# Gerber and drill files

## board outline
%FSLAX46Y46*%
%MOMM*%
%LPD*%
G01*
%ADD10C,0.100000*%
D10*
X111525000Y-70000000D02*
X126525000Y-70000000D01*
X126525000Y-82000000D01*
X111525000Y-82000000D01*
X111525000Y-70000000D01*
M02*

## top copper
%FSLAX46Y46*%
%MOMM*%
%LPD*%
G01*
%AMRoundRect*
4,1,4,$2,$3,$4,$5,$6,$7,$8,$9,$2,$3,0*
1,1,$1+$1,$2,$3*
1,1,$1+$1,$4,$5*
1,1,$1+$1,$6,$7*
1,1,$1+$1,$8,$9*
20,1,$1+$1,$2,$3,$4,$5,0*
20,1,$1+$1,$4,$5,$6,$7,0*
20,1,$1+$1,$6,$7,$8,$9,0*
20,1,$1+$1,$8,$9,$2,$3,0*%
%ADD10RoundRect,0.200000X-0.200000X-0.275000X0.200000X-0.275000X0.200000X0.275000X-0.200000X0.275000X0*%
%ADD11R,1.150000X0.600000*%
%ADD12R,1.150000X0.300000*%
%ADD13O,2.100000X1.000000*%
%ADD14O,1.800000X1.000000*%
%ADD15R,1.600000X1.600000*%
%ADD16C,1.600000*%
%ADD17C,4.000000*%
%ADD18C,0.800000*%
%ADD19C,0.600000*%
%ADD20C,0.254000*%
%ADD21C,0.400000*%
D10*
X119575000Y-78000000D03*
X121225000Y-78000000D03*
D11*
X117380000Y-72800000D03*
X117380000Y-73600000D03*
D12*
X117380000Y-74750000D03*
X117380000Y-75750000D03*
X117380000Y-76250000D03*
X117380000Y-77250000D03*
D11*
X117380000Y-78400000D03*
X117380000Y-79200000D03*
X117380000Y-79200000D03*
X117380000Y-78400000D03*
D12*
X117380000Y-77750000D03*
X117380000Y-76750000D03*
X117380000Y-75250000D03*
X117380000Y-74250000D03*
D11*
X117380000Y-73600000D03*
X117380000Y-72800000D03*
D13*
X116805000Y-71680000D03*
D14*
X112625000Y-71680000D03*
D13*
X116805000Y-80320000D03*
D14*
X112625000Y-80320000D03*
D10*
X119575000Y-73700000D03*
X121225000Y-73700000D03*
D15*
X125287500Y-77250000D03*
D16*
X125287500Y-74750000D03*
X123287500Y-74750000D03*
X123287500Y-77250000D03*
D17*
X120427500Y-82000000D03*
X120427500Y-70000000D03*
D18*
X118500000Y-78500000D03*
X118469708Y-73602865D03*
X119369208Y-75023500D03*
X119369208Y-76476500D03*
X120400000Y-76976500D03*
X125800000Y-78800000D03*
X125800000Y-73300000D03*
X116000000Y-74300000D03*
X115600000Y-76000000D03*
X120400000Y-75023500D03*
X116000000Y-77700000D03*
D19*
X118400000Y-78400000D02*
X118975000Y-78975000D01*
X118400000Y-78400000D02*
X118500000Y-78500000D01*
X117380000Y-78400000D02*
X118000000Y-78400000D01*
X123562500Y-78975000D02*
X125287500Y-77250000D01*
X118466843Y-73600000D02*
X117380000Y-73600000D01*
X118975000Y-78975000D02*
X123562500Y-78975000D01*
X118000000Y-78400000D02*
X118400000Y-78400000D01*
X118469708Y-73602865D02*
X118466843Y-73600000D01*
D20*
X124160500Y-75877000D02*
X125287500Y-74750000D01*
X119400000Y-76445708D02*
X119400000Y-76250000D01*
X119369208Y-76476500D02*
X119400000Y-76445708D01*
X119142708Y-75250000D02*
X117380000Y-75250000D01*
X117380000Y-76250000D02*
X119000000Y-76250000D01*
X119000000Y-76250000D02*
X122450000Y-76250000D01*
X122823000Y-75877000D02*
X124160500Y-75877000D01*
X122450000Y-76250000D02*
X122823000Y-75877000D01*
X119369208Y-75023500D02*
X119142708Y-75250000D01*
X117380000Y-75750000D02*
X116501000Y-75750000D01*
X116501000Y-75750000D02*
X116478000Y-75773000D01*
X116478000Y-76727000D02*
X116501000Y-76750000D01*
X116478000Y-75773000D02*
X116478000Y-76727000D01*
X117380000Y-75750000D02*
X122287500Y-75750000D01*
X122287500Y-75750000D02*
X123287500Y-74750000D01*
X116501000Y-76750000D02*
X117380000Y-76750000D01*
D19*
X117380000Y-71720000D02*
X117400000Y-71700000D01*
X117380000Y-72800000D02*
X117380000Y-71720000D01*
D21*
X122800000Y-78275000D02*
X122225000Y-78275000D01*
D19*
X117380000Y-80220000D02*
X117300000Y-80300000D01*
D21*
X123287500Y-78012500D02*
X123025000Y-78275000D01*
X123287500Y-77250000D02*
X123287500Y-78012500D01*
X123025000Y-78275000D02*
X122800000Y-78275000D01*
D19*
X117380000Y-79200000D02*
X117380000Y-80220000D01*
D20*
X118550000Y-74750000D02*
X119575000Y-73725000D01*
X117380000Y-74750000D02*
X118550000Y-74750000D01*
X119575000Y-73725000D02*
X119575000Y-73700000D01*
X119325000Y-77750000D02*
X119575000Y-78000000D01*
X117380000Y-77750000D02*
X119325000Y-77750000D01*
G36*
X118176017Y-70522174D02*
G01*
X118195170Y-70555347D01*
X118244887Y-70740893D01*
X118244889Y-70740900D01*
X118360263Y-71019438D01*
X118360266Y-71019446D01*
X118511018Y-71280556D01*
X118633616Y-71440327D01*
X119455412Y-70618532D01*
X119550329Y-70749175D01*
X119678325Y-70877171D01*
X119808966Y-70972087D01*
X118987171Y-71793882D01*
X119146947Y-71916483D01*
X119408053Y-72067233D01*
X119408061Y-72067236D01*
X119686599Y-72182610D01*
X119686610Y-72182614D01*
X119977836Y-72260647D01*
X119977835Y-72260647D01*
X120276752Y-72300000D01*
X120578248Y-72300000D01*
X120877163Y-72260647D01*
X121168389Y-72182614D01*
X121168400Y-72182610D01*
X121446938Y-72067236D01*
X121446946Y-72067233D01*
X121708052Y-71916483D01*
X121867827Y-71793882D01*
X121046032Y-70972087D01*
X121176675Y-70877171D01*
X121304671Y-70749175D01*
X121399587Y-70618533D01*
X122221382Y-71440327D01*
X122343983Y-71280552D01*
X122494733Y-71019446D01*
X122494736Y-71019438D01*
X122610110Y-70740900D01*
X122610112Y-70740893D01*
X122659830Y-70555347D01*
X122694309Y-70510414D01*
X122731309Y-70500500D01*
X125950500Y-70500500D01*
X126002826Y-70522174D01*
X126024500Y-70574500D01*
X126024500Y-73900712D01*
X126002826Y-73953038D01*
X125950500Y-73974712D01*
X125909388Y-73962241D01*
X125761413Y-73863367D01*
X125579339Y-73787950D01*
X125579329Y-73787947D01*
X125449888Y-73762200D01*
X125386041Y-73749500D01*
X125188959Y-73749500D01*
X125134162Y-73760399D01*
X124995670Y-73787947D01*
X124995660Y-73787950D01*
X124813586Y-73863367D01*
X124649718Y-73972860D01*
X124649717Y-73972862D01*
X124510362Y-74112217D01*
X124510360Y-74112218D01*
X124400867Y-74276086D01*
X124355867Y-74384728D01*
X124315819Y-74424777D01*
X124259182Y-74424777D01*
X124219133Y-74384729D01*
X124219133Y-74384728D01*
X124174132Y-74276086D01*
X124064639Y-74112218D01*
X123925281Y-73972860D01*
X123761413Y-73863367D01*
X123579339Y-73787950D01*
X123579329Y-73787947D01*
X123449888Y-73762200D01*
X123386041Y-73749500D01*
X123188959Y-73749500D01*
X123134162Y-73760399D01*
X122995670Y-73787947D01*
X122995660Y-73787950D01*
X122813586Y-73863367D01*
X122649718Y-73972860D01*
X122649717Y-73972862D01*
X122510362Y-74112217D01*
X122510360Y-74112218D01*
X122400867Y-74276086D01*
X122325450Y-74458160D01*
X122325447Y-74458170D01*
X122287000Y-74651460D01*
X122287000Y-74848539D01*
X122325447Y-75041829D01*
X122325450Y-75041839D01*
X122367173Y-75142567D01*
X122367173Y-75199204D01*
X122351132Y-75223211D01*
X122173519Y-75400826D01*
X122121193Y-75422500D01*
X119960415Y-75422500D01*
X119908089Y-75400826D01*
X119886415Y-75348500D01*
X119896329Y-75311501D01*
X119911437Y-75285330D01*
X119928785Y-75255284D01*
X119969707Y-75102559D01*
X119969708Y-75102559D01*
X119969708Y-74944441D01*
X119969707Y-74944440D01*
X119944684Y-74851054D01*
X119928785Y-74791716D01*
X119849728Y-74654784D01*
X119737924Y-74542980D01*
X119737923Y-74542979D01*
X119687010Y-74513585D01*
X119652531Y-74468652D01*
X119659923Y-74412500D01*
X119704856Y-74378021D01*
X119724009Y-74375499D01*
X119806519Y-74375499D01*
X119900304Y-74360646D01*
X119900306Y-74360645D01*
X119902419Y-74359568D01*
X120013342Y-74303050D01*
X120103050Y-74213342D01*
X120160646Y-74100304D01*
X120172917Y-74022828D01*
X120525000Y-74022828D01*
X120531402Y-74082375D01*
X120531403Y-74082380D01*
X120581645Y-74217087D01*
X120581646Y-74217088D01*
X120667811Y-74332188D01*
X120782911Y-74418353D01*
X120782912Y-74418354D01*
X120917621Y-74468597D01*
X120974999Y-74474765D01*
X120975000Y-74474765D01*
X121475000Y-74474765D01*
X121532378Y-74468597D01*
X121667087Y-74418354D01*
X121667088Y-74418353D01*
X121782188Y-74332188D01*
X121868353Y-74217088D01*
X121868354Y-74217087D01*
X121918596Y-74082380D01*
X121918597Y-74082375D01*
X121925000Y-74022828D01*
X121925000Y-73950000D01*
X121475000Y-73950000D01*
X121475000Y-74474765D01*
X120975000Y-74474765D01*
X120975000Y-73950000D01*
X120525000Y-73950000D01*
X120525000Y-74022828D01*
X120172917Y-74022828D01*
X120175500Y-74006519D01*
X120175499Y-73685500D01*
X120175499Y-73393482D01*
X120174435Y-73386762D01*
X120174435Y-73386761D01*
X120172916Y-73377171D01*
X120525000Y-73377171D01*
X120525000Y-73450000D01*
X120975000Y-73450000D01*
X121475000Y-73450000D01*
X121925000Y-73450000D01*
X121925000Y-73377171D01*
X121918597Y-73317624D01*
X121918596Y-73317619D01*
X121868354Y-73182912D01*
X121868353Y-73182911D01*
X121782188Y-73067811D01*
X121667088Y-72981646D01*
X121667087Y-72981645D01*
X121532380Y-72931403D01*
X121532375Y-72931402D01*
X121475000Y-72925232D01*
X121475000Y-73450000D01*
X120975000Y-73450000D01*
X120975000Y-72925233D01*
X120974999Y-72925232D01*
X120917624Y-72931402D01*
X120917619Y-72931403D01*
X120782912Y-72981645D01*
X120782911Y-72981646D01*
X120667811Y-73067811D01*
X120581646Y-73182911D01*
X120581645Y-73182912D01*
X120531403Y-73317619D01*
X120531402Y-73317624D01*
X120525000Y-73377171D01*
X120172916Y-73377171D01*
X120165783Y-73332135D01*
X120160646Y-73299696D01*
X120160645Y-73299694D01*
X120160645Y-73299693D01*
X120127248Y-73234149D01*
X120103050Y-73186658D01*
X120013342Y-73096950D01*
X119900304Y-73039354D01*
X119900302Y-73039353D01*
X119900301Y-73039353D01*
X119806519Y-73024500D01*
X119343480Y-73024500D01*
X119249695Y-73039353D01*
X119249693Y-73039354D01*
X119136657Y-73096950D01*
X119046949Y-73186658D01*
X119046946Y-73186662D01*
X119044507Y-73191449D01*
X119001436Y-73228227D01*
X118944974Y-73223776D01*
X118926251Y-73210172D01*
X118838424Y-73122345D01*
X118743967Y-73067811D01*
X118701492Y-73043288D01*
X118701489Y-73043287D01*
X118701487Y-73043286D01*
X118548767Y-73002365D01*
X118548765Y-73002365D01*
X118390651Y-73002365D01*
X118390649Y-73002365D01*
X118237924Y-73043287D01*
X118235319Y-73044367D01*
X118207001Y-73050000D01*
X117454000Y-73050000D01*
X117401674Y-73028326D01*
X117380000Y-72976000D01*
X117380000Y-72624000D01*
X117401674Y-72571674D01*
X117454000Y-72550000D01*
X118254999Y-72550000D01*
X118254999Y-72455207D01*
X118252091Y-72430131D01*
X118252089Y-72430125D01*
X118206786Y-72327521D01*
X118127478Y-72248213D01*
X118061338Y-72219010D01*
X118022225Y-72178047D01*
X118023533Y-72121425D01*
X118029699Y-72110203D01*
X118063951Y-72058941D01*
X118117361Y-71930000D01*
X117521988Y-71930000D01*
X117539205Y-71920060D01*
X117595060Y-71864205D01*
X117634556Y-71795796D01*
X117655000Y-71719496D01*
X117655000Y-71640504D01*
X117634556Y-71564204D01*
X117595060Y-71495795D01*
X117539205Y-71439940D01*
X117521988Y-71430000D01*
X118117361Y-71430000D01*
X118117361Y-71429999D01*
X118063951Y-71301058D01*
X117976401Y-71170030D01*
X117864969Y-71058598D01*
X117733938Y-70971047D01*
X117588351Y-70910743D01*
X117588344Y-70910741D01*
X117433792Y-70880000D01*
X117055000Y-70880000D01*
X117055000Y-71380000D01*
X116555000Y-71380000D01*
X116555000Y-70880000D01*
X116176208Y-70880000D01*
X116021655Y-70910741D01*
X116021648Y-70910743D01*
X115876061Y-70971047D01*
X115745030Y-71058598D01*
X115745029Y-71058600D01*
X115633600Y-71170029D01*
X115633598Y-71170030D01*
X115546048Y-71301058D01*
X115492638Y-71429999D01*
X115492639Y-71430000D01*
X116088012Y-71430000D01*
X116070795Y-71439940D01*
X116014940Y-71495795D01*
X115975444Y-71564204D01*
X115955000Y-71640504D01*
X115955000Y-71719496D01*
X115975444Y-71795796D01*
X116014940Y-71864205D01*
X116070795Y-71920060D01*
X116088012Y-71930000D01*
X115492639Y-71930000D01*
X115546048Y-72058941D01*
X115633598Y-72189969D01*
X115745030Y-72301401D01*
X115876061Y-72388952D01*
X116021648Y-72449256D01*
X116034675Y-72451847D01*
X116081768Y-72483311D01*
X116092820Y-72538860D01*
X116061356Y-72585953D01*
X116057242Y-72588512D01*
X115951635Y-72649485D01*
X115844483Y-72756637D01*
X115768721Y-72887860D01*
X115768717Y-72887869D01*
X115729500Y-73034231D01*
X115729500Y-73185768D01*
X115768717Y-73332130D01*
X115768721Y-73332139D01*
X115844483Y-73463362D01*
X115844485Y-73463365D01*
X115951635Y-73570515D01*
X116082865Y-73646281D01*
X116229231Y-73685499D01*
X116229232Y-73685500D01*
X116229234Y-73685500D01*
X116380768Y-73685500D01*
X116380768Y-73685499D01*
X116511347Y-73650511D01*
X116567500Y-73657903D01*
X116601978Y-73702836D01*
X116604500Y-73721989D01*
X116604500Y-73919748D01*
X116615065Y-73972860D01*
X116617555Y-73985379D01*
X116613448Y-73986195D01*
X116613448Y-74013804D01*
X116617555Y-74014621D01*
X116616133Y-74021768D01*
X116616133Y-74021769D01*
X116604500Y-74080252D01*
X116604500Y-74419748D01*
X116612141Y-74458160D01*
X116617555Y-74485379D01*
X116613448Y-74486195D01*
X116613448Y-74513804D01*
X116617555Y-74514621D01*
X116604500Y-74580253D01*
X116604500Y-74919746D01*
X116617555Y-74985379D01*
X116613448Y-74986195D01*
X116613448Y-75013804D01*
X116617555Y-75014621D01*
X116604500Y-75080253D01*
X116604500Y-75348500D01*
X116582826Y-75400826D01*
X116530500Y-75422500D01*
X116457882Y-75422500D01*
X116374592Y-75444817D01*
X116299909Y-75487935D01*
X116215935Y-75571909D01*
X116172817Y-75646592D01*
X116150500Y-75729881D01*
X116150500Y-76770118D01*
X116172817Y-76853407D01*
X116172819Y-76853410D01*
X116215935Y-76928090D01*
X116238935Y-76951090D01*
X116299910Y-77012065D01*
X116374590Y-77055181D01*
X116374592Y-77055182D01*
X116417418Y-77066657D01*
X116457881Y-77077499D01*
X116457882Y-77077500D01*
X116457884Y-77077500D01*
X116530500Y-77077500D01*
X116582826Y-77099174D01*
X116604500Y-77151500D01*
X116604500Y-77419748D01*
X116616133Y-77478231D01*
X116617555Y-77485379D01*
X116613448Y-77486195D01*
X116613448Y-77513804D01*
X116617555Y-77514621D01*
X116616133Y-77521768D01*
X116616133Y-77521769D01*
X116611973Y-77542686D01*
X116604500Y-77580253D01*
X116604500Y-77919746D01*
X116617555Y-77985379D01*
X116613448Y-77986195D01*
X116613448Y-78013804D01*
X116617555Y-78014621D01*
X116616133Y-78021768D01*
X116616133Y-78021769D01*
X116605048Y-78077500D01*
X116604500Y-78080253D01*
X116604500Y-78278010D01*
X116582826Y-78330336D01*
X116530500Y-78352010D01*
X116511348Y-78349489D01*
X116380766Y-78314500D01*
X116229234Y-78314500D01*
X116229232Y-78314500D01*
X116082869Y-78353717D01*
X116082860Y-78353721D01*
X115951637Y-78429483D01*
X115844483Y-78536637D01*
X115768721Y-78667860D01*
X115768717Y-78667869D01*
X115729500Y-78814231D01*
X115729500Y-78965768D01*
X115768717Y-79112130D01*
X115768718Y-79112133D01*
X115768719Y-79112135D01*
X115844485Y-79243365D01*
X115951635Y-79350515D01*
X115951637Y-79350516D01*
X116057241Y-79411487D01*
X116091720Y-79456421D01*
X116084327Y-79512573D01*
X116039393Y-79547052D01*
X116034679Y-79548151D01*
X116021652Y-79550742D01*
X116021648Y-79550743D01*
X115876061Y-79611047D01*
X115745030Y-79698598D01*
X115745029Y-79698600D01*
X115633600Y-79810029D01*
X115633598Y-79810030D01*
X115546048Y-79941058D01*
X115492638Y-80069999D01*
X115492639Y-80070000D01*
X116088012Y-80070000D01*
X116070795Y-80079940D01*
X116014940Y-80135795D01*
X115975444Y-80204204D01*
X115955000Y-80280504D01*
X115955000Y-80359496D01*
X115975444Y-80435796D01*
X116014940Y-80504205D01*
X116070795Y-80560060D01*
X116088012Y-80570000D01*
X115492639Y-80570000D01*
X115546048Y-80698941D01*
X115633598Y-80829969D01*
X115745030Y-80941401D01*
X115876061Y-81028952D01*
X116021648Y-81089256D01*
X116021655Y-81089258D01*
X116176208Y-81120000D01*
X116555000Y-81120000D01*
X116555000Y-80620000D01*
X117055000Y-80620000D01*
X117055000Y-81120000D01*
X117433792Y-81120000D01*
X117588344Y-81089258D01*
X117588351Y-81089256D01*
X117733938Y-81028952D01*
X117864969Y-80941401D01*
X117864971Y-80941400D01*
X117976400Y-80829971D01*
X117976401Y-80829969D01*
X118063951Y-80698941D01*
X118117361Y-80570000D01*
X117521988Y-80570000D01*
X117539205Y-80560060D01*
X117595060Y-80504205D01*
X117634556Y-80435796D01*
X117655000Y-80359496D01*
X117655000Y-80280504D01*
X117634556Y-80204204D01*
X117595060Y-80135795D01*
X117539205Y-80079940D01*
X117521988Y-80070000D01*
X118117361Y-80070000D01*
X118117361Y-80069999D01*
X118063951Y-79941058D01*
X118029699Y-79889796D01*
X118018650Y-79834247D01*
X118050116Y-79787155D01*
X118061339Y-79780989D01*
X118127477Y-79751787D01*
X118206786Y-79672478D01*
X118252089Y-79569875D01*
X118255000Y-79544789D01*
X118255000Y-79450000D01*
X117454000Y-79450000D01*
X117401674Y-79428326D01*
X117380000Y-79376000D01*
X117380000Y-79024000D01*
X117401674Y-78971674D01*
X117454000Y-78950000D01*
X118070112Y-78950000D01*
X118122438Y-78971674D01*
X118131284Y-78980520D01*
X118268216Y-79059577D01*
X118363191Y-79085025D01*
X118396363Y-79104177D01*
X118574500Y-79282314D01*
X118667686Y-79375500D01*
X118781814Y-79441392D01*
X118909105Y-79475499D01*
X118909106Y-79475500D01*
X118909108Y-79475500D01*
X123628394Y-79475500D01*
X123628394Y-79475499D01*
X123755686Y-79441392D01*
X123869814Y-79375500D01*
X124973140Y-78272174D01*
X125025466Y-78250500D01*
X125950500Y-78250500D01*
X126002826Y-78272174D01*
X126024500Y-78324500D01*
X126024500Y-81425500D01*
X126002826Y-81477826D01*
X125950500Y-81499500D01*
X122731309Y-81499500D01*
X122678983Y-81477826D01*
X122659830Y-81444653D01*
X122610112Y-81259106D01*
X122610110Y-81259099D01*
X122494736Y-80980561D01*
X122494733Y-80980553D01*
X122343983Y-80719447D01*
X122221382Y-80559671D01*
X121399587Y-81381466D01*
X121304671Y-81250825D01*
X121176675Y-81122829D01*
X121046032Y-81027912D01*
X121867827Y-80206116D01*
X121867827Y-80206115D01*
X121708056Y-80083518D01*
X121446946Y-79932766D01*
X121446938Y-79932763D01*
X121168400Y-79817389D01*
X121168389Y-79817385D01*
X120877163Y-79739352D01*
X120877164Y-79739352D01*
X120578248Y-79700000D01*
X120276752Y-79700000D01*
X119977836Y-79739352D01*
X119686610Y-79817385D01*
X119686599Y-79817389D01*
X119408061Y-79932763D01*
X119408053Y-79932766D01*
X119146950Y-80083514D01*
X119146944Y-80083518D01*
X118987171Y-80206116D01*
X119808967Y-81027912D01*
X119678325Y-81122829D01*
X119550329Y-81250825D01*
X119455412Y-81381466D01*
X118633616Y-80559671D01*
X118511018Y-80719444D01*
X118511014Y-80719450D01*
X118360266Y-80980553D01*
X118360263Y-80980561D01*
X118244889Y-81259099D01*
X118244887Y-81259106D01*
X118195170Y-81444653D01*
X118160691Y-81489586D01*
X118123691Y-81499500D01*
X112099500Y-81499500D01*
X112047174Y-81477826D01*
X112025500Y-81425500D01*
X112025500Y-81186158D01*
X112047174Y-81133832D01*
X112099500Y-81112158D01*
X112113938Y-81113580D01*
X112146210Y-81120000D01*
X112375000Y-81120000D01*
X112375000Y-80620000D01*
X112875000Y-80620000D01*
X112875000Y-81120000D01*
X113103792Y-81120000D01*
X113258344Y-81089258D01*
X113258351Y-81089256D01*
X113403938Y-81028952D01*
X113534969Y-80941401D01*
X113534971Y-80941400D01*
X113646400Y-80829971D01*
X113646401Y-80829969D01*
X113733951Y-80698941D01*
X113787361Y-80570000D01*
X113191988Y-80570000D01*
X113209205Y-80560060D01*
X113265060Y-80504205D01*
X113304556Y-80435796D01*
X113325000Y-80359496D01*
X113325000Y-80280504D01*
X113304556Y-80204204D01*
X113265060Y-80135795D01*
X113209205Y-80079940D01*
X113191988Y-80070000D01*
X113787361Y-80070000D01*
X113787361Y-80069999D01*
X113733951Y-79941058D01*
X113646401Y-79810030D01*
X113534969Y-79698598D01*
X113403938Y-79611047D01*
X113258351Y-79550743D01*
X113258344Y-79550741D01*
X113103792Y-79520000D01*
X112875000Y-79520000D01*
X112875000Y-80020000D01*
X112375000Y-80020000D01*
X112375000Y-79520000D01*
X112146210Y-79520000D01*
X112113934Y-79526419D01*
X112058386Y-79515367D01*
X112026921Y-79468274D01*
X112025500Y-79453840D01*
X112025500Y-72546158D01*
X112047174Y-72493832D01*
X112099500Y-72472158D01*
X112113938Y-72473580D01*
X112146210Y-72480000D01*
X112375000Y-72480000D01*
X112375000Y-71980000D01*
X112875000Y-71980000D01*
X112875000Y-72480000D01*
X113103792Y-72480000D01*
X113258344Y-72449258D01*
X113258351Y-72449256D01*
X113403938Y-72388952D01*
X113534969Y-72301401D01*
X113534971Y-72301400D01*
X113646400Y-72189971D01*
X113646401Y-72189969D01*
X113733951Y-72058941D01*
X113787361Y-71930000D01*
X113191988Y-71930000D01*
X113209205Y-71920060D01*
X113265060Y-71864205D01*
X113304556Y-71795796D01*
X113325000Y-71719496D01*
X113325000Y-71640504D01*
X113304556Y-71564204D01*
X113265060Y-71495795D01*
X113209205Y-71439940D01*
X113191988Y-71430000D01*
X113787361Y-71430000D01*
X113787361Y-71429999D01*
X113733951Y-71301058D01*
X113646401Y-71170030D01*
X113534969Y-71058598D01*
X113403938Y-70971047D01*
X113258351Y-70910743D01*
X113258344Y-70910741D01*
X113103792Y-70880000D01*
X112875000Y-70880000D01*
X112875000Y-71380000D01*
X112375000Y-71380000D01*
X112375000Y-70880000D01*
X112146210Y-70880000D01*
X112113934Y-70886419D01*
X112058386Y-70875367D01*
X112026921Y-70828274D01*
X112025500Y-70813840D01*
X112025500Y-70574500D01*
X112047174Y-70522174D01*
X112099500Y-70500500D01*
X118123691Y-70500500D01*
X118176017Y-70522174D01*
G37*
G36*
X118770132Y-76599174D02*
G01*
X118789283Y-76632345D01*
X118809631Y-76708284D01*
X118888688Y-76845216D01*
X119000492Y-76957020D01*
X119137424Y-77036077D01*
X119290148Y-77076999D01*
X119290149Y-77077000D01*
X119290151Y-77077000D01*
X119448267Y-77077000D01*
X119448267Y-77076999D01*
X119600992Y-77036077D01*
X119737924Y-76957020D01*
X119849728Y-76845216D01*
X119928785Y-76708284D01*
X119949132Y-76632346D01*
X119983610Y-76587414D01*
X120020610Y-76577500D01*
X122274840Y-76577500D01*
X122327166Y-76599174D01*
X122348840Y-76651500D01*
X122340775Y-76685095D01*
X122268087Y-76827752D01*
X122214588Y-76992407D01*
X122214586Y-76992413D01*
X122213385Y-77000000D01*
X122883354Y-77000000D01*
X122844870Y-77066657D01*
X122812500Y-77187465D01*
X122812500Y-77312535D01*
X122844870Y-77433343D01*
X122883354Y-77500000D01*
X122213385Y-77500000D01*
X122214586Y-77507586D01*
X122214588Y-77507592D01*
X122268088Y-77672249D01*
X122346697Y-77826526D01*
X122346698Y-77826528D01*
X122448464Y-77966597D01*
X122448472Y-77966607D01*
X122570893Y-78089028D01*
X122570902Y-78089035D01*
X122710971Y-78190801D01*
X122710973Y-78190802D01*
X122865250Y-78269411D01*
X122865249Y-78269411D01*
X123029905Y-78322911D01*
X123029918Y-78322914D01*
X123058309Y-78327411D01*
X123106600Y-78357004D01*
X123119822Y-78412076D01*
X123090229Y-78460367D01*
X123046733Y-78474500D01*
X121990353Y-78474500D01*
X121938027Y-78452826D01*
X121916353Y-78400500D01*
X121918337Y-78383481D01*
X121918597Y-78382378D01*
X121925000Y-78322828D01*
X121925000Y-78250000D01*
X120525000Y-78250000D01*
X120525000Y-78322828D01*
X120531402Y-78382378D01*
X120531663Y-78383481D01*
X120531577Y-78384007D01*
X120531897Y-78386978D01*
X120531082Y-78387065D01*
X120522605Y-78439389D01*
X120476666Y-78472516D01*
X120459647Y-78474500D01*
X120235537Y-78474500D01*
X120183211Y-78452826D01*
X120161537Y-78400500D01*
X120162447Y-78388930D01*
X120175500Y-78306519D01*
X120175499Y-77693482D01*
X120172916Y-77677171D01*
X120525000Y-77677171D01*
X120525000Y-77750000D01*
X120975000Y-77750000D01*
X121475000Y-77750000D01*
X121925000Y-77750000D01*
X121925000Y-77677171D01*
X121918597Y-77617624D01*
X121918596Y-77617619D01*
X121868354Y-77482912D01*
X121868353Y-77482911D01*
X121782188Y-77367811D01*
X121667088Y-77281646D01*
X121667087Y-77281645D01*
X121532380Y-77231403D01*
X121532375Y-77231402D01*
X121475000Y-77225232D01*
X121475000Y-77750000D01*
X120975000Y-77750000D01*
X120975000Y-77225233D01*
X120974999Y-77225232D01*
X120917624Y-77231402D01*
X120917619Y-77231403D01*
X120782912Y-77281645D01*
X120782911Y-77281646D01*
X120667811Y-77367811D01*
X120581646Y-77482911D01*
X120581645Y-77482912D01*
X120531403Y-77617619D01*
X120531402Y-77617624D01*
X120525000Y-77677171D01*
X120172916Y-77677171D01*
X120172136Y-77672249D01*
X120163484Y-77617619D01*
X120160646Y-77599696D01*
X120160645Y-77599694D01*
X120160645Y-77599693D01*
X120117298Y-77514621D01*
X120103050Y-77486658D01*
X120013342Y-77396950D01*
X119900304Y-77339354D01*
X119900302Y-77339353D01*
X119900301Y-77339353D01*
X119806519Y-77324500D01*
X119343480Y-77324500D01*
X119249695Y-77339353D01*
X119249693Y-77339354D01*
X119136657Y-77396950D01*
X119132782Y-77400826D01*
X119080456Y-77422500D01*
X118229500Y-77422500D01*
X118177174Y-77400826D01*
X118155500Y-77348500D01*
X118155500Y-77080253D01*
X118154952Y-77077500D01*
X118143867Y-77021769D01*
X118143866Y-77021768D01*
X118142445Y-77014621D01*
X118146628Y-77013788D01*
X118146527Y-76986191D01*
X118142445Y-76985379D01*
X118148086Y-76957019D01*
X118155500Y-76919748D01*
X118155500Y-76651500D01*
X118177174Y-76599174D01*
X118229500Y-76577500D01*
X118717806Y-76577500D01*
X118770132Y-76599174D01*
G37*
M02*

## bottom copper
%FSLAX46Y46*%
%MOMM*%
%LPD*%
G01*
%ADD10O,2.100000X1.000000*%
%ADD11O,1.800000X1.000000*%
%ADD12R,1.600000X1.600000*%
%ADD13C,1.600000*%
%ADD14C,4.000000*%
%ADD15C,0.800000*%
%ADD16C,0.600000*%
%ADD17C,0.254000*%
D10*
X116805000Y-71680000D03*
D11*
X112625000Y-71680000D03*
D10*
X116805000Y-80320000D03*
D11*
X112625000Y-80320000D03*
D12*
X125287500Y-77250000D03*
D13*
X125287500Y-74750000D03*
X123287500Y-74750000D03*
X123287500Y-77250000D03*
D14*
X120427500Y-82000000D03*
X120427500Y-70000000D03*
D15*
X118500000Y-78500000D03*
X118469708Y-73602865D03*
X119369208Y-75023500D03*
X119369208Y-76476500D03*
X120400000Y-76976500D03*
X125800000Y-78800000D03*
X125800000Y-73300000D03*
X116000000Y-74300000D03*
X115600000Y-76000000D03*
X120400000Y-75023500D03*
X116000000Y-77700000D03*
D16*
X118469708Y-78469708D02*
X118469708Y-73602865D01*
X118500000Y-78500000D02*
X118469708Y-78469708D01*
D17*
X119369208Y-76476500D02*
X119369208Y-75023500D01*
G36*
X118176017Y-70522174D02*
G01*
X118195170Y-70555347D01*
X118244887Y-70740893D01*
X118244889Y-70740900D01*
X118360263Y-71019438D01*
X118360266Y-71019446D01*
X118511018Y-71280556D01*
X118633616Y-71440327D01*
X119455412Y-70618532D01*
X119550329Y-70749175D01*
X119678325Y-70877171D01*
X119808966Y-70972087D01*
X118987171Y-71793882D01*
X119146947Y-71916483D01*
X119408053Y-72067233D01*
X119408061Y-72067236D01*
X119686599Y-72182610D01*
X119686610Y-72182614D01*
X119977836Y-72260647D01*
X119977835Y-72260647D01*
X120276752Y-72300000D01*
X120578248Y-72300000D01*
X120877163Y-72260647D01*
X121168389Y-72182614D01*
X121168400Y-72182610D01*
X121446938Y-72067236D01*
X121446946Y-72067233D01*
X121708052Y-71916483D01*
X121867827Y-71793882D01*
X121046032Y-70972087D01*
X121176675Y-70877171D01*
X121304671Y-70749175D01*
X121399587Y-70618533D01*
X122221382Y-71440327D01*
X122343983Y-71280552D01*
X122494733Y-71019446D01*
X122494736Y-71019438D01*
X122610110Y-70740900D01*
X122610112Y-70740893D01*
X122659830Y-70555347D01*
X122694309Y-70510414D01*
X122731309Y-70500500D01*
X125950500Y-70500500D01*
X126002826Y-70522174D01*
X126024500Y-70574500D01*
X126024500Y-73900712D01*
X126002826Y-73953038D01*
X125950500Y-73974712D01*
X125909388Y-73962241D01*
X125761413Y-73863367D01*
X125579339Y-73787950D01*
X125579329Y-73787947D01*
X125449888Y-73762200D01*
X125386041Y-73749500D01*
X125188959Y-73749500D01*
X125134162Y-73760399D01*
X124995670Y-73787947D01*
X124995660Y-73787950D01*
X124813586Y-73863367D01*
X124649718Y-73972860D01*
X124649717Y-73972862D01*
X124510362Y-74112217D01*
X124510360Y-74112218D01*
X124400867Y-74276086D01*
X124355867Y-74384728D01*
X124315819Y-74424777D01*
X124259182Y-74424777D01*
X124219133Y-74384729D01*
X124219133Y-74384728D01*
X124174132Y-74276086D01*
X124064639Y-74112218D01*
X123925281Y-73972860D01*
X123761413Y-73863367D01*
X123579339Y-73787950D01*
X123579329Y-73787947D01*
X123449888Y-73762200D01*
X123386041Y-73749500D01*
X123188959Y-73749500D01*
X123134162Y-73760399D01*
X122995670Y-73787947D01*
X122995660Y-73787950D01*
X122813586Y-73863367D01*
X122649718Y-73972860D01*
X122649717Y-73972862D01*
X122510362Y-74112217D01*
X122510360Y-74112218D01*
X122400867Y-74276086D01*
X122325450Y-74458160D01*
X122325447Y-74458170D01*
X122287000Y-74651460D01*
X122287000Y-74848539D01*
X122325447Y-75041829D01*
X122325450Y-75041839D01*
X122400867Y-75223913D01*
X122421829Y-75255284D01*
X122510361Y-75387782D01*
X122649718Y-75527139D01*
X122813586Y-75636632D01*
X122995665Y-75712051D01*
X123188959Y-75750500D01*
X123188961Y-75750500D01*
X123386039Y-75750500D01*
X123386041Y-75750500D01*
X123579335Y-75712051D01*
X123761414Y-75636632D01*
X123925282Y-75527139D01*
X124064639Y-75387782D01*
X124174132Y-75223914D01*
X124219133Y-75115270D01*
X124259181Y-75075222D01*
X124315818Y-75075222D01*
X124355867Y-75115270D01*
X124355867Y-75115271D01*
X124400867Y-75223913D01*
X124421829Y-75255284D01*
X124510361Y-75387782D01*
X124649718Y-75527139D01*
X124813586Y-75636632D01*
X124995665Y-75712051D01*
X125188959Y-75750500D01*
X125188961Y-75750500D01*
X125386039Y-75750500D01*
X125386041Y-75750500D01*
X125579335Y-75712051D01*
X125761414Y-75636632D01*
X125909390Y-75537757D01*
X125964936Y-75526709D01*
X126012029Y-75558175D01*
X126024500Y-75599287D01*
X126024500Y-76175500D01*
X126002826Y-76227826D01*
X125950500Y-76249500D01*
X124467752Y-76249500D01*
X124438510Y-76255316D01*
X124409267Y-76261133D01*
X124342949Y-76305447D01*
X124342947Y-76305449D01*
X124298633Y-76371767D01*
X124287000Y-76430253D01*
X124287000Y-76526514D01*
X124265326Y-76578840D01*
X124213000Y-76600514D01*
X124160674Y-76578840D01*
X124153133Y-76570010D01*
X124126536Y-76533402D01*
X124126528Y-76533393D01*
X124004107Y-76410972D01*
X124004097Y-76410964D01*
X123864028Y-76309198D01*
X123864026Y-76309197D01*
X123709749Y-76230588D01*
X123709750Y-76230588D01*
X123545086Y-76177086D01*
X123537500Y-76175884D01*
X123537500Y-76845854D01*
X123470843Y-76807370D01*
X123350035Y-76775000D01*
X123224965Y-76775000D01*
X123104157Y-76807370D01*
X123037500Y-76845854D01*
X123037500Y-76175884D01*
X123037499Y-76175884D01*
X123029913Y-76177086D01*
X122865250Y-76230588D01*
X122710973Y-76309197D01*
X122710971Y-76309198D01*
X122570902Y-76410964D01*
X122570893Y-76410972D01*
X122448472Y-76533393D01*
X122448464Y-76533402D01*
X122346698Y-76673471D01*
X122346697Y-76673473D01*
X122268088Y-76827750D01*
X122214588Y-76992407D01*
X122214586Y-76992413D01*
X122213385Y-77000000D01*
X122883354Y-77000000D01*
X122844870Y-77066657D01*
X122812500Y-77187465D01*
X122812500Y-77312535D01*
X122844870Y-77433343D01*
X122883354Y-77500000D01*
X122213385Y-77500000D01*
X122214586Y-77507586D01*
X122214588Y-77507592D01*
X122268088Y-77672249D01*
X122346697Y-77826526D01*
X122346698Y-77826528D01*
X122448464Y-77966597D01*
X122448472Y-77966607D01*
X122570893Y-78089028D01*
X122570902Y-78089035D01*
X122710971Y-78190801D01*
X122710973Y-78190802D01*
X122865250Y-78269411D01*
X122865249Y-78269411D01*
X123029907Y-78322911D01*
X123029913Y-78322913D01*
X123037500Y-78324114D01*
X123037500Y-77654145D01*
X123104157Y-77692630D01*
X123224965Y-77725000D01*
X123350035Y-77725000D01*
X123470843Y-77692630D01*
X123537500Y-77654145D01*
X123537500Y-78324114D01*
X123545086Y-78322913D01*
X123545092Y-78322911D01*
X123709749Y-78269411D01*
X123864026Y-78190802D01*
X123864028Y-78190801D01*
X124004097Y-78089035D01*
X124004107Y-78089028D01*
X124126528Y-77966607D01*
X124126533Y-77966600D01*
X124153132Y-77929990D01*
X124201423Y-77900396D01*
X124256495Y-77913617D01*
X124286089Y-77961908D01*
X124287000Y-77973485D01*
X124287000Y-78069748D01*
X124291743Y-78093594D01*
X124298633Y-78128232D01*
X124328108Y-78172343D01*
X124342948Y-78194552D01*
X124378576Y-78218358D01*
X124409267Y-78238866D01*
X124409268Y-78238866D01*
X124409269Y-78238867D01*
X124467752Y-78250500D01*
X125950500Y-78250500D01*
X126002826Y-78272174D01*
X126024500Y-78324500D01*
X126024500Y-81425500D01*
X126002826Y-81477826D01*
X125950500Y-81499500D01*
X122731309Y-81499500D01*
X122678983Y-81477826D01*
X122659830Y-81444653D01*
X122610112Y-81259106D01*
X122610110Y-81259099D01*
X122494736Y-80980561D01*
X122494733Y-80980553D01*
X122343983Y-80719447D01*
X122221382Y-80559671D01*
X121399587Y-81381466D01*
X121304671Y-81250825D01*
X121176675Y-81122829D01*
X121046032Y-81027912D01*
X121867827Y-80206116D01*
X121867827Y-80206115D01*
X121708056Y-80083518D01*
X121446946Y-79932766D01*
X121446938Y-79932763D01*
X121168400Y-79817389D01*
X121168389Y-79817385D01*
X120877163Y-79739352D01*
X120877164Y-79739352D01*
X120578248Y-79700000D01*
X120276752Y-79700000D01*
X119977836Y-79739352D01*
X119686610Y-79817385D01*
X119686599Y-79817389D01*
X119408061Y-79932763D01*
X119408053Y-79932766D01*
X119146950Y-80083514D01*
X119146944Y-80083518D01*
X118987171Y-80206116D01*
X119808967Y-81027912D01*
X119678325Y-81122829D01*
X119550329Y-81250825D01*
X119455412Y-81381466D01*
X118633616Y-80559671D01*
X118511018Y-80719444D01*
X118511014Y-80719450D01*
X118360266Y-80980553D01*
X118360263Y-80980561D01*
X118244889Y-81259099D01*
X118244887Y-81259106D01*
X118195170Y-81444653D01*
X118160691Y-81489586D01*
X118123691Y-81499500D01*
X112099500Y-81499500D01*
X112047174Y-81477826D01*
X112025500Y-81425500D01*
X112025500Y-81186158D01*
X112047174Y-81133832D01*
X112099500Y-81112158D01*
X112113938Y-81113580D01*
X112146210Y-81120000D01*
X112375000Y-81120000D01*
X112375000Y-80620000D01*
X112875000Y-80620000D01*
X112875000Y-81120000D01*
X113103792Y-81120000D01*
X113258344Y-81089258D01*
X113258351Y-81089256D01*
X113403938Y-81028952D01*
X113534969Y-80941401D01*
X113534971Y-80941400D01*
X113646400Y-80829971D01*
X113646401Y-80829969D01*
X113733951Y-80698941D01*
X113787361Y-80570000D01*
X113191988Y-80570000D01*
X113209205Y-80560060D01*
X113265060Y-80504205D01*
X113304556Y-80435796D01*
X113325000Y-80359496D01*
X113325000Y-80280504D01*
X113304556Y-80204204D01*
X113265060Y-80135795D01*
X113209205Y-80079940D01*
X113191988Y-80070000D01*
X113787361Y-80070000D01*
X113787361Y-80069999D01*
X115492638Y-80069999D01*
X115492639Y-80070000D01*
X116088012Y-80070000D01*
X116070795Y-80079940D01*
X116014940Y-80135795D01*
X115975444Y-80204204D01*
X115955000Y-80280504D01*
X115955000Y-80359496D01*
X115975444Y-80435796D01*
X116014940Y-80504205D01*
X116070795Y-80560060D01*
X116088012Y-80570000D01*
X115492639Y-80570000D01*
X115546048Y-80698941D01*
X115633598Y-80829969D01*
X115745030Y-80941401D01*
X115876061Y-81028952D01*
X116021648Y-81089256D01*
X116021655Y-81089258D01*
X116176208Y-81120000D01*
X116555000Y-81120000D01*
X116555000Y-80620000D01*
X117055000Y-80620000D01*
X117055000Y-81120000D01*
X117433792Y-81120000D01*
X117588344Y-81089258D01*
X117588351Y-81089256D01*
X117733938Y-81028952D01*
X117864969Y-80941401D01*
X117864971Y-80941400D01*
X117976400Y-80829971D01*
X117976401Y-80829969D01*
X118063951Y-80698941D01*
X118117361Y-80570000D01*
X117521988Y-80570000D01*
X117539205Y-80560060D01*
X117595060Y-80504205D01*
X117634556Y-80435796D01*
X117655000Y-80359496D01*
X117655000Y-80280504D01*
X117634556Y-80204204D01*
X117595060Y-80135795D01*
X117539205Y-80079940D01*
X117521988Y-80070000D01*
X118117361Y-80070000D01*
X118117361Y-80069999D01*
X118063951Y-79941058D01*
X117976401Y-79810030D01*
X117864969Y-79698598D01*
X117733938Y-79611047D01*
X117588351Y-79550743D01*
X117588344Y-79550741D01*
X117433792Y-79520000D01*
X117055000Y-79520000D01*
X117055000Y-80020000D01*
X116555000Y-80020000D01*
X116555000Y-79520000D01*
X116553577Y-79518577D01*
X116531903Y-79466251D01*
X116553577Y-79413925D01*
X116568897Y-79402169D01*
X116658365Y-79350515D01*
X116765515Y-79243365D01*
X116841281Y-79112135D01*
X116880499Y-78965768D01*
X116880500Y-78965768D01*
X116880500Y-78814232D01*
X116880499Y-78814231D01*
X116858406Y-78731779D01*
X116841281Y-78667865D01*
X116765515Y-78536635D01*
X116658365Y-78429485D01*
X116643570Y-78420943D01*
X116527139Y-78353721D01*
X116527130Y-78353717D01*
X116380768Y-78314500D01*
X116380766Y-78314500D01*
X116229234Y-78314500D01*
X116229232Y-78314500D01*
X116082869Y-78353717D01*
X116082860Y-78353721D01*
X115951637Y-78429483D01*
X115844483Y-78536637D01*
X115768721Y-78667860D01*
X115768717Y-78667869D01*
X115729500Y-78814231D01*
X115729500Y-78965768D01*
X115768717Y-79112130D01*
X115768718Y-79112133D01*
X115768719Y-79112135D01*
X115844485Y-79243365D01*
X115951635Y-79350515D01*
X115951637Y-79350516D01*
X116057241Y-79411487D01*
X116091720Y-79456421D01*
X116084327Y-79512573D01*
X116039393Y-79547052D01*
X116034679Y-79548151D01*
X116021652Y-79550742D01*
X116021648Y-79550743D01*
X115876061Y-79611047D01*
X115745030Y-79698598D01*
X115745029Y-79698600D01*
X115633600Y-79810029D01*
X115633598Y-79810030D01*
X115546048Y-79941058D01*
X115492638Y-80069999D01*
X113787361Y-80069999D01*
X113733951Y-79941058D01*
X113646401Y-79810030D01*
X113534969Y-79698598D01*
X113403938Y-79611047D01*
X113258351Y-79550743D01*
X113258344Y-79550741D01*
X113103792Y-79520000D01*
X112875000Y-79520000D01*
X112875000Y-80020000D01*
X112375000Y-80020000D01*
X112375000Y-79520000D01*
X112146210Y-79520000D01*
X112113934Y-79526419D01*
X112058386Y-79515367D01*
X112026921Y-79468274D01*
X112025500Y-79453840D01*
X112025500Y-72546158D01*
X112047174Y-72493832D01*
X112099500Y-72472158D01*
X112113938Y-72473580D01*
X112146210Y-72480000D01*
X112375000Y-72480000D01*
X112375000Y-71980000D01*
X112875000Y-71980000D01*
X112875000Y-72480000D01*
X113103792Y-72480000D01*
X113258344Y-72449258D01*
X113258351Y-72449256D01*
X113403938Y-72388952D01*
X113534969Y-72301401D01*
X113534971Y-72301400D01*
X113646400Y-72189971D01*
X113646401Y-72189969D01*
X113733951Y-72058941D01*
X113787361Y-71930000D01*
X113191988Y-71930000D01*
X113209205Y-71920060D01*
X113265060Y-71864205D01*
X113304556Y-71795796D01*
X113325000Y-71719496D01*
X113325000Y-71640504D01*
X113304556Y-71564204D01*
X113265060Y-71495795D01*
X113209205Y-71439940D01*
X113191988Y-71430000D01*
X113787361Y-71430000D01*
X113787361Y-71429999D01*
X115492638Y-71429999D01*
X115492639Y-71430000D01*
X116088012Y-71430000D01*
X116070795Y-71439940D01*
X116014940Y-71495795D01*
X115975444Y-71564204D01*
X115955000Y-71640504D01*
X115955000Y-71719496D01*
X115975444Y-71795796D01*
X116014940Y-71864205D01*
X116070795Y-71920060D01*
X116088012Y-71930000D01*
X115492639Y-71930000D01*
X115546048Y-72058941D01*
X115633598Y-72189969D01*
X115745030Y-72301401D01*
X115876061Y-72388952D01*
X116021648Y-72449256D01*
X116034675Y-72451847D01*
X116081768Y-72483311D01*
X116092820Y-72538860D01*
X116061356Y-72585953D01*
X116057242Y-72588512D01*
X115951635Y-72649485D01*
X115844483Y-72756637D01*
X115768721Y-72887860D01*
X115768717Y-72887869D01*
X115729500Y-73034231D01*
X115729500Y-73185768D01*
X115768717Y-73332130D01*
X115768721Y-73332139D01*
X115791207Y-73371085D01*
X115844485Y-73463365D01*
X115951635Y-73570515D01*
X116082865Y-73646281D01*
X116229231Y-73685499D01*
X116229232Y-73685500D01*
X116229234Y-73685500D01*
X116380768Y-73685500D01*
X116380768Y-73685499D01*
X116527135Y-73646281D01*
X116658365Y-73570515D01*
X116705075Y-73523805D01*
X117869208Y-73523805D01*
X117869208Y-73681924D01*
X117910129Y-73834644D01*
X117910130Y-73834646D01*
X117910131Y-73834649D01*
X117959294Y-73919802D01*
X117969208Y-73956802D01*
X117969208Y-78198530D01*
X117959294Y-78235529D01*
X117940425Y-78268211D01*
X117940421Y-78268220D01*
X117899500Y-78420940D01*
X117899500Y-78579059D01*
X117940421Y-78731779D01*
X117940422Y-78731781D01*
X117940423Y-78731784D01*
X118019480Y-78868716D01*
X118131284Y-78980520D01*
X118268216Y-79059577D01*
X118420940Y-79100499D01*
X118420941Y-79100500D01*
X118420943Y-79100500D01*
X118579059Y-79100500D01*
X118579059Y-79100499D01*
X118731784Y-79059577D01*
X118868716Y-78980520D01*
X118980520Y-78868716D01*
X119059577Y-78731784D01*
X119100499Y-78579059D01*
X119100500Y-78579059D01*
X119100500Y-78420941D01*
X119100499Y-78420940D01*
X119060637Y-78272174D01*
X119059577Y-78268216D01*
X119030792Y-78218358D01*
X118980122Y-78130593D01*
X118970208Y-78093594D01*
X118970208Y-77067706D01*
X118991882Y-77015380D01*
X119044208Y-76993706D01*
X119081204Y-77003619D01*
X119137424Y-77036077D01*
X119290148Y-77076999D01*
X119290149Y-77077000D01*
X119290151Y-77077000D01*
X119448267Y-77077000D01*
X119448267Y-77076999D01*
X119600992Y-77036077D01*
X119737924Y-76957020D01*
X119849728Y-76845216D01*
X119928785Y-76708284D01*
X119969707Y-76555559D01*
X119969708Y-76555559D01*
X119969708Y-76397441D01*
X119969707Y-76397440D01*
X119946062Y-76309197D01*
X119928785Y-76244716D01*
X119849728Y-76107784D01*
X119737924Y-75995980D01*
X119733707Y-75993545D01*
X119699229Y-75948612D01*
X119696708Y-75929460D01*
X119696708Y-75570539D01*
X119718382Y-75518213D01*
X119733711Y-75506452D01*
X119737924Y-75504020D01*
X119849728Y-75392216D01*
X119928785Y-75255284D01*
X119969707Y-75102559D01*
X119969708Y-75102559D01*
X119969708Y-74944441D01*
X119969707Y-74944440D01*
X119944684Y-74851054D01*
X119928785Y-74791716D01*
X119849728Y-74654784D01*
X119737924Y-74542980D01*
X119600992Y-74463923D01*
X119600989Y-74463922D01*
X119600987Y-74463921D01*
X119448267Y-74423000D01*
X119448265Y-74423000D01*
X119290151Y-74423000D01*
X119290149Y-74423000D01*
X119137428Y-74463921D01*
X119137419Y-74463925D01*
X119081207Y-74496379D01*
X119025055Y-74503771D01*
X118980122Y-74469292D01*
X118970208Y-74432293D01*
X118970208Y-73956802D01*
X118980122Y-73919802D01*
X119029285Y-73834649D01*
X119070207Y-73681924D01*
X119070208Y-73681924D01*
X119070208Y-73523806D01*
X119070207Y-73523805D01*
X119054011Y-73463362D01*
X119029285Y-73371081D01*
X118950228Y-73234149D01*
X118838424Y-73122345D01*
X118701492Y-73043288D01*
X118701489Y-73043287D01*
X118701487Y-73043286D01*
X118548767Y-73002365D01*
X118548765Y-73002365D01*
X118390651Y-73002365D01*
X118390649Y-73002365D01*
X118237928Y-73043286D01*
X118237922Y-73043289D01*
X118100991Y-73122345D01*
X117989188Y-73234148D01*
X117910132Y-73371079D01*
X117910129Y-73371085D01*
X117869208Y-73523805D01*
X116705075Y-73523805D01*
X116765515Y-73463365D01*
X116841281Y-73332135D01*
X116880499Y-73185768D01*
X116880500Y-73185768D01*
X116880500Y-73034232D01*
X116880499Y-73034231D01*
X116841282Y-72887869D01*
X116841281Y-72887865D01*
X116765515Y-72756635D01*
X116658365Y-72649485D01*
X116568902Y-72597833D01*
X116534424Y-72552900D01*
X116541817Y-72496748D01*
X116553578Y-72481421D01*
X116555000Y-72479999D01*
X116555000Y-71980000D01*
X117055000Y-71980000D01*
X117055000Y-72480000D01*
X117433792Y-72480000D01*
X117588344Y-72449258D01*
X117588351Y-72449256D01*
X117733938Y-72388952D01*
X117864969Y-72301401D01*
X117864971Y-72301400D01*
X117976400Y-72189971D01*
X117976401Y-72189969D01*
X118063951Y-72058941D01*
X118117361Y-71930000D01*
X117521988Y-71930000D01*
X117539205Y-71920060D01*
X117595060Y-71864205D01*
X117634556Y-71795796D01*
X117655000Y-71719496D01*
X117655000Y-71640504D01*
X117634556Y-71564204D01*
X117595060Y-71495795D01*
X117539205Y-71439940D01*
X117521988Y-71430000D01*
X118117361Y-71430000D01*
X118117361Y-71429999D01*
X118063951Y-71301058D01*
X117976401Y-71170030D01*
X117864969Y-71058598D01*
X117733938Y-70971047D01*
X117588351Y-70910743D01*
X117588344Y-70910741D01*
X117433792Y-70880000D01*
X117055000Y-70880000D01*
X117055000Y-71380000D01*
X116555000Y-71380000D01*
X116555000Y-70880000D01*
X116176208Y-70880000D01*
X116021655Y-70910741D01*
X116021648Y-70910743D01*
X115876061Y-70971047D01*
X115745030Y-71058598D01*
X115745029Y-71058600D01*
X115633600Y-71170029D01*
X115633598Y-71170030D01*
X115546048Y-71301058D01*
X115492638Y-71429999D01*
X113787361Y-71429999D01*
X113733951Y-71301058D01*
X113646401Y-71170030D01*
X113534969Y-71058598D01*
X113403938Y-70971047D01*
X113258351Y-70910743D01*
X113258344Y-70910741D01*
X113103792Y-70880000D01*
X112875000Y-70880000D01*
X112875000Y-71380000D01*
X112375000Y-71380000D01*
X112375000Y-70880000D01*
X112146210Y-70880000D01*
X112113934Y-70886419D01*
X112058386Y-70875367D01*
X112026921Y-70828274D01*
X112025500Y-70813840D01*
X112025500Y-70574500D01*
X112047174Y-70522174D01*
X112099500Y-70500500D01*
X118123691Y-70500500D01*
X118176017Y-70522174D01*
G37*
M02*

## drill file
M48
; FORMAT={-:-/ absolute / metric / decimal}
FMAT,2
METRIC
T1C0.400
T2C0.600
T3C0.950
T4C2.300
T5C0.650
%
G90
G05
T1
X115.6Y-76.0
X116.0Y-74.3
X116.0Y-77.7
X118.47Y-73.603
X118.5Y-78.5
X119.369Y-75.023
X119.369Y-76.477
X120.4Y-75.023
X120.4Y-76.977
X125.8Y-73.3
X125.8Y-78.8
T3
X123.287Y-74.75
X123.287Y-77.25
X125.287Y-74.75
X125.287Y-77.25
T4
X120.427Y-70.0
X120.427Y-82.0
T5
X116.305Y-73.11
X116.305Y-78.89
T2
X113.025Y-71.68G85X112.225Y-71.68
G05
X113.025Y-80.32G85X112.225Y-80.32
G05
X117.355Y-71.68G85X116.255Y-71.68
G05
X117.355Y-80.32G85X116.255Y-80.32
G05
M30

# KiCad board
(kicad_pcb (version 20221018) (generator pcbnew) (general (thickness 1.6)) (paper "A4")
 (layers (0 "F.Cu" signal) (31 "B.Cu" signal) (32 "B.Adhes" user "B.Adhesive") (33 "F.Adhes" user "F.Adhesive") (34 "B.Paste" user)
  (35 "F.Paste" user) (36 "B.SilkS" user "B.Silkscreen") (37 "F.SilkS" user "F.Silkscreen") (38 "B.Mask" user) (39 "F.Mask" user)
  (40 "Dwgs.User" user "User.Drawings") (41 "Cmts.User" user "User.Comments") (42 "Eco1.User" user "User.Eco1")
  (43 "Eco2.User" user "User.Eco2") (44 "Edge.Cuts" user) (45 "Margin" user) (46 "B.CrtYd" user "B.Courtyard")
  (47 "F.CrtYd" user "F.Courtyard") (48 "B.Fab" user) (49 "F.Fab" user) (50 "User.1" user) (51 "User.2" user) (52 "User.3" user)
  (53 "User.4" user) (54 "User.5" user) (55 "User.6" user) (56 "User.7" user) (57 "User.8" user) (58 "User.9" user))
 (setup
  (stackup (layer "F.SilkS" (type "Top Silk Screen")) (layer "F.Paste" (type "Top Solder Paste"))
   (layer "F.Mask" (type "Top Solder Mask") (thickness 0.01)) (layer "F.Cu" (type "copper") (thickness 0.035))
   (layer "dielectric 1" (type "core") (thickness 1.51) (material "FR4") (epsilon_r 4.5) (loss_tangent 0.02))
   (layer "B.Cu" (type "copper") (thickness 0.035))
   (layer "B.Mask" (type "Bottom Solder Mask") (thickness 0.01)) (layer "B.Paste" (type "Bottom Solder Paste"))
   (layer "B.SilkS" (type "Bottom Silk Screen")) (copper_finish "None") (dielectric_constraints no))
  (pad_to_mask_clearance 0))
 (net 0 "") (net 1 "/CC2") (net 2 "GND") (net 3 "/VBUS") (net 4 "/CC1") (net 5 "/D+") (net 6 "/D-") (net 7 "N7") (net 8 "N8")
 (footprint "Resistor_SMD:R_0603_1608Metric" (layer "F.Cu") (at 120.4 78)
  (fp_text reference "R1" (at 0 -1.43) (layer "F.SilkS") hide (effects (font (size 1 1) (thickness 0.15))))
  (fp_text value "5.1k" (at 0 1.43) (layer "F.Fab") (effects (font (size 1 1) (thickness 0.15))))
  (pad "1" smd roundrect (at -0.825 0) (size 0.8 0.95) (layers "F.Cu" "F.Paste" "F.Mask") (roundrect_rratio 0.25) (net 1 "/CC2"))
  (pad "2" smd roundrect (at 0.825 0) (size 0.8 0.95) (layers "F.Cu" "F.Paste" "F.Mask") (roundrect_rratio 0.25) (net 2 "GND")))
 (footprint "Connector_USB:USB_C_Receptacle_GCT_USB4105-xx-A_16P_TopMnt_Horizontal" (layer "F.Cu") (at 113.7 76 -90)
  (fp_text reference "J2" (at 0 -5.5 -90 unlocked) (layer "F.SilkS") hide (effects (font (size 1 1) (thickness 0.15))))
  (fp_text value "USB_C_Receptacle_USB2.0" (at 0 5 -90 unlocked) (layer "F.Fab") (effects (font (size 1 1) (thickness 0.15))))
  (pad "" np_thru_hole circle (at -2.89 -2.605 270) (size 0.65 0.65) (drill 0.65) (layers "F&B.Cu" "*.Mask"))
  (pad "" np_thru_hole circle (at 2.89 -2.605 270) (size 0.65 0.65) (drill 0.65) (layers "F&B.Cu" "*.Mask"))
  (pad "A1" smd rect (at -3.2 -3.68 270) (size 0.6 1.15) (layers "F.Cu" "F.Paste" "F.Mask") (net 2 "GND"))
  (pad "A4" smd rect (at -2.4 -3.68 270) (size 0.6 1.15) (layers "F.Cu" "F.Paste" "F.Mask") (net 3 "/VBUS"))
  (pad "A5" smd rect (at -1.25 -3.68 270) (size 0.3 1.15) (layers "F.Cu" "F.Paste" "F.Mask") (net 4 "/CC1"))
  (pad "A6" smd rect (at -0.25 -3.68 270) (size 0.3 1.15) (layers "F.Cu" "F.Paste" "F.Mask") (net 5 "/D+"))
  (pad "A7" smd rect (at 0.25 -3.68 270) (size 0.3 1.15) (layers "F.Cu" "F.Paste" "F.Mask") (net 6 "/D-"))
  (pad "A8" smd rect (at 1.25 -3.68 270) (size 0.3 1.15) (layers "F.Cu" "F.Paste" "F.Mask") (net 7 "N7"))
  (pad "A9" smd rect (at 2.4 -3.68 270) (size 0.6 1.15) (layers "F.Cu" "F.Paste" "F.Mask") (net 3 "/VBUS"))
  (pad "A12" smd rect (at 3.2 -3.68 270) (size 0.6 1.15) (layers "F.Cu" "F.Paste" "F.Mask") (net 2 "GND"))
  (pad "B1" smd rect (at 3.2 -3.68 270) (size 0.6 1.15) (layers "F.Cu" "F.Paste" "F.Mask") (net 2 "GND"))
  (pad "B4" smd rect (at 2.4 -3.68 270) (size 0.6 1.15) (layers "F.Cu" "F.Paste" "F.Mask") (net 3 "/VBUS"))
  (pad "B5" smd rect (at 1.75 -3.68 270) (size 0.3 1.15) (layers "F.Cu" "F.Paste" "F.Mask") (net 1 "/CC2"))
  (pad "B6" smd rect (at 0.75 -3.68 270) (size 0.3 1.15) (layers "F.Cu" "F.Paste" "F.Mask") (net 5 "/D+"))
  (pad "B7" smd rect (at -0.75 -3.68 270) (size 0.3 1.15) (layers "F.Cu" "F.Paste" "F.Mask") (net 6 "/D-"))
  (pad "B8" smd rect (at -1.75 -3.68 270) (size 0.3 1.15) (layers "F.Cu" "F.Paste" "F.Mask") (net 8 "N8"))
  (pad "B9" smd rect (at -2.4 -3.68 270) (size 0.6 1.15) (layers "F.Cu" "F.Paste" "F.Mask") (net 3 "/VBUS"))
  (pad "B12" smd rect (at -3.2 -3.68 270) (size 0.6 1.15) (layers "F.Cu" "F.Paste" "F.Mask") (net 2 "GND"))
  (pad "S1" thru_hole oval (at -4.32 -3.105 270) (size 1 2.1) (drill oval 0.6 1.7) (layers "*.Cu" "*.Mask") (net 2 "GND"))
  (pad "S1" thru_hole oval (at -4.32 1.075 270) (size 1 1.8) (drill oval 0.6 1.4) (layers "*.Cu" "*.Mask") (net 2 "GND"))
  (pad "S1" thru_hole oval (at 4.32 -3.105 270) (size 1 2.1) (drill oval 0.6 1.7) (layers "*.Cu" "*.Mask") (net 2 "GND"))
  (pad "S1" thru_hole oval (at 4.32 1.075 270) (size 1 1.8) (drill oval 0.6 1.4) (layers "*.Cu" "*.Mask") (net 2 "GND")))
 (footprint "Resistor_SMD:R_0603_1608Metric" (layer "F.Cu") (at 120.4 73.7)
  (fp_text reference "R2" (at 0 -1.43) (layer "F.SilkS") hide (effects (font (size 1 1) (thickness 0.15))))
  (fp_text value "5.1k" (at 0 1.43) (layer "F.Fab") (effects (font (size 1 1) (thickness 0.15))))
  (pad "1" smd roundrect (at -0.825 0) (size 0.8 0.95) (layers "F.Cu" "F.Paste" "F.Mask") (roundrect_rratio 0.25) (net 4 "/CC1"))
  (pad "2" smd roundrect (at 0.825 0) (size 0.8 0.95) (layers "F.Cu" "F.Paste" "F.Mask") (roundrect_rratio 0.25) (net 2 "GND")))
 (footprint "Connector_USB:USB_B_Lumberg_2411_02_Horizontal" (layer "F.Cu") (at 125.2875 77.25 180)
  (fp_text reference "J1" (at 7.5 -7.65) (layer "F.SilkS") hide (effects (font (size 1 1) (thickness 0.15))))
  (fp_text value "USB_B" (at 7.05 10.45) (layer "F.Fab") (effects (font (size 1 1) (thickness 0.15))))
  (pad "1" thru_hole rect (at 0 0 270) (size 1.6 1.6) (drill 0.95) (layers "*.Cu" "*.Mask") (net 3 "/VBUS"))
  (pad "2" thru_hole circle (at 0 2.5 270) (size 1.6 1.6) (drill 0.95) (layers "*.Cu" "*.Mask") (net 6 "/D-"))
  (pad "3" thru_hole circle (at 2 2.5 270) (size 1.6 1.6) (drill 0.95) (layers "*.Cu" "*.Mask") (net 5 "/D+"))
  (pad "4" thru_hole circle (at 2 0 270) (size 1.6 1.6) (drill 0.95) (layers "*.Cu" "*.Mask") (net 2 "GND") (thermal_bridge_angle 0))
  (pad "5" thru_hole circle (at 4.86 -4.75 270) (size 4 4) (drill 2.3) (layers "*.Cu" "*.Mask") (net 2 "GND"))
  (pad "5" thru_hole circle (at 4.86 7.25 270) (size 4 4) (drill 2.3) (layers "*.Cu" "*.Mask") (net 2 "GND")))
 (gr_rect (start 111.525 70) (end 126.525 82) (stroke (width 0.1) (type default)) (fill none) (layer "Edge.Cuts"))
 (segment (start 118.4 78.4) (end 118.975 78.975) (width 0.6) (layer "F.Cu") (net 3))
 (segment (start 118.4 78.4) (end 118.5 78.5) (width 0.6) (layer "F.Cu") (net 3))
 (segment (start 117.38 78.4) (end 118 78.4) (width 0.6) (layer "F.Cu") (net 3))
 (segment (start 123.5625 78.975) (end 125.2875 77.25) (width 0.6) (layer "F.Cu") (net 3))
 (segment (start 118.466843 73.6) (end 117.38 73.6) (width 0.6) (layer "F.Cu") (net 3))
 (segment (start 118.975 78.975) (end 123.5625 78.975) (width 0.6) (layer "F.Cu") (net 3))
 (segment (start 118 78.4) (end 118.4 78.4) (width 0.6) (layer "F.Cu") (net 3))
 (segment (start 118.469708 73.602865) (end 118.466843 73.6) (width 0.6) (layer "F.Cu") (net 3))
 (via (at 118.5 78.5) (size 0.8) (drill 0.4) (layers "F.Cu" "B.Cu") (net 3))
 (via (at 118.469708 73.602865) (size 0.8) (drill 0.4) (layers "F.Cu" "B.Cu") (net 3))
 (segment (start 118.469708 78.469708) (end 118.469708 73.602865) (width 0.6) (layer "B.Cu") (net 3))
 (segment (start 118.5 78.5) (end 118.469708 78.469708) (width 0.6) (layer "B.Cu") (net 3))
 (segment (start 124.1605 75.877) (end 125.2875 74.75) (width 0.254) (layer "F.Cu") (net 6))
 (segment (start 119.4 76.445708) (end 119.4 76.25) (width 0.254) (layer "F.Cu") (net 6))
 (segment (start 119.369208 76.4765) (end 119.4 76.445708) (width 0.254) (layer "F.Cu") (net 6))
 (segment (start 119.142708 75.25) (end 117.38 75.25) (width 0.254) (layer "F.Cu") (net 6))
 (segment (start 117.38 76.25) (end 119 76.25) (width 0.254) (layer "F.Cu") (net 6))
 (segment (start 119 76.25) (end 122.45 76.25) (width 0.254) (layer "F.Cu") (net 6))
 (segment (start 122.823 75.877) (end 124.1605 75.877) (width 0.254) (layer "F.Cu") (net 6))
 (segment (start 122.45 76.25) (end 122.823 75.877) (width 0.254) (layer "F.Cu") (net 6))
 (segment (start 119.369208 75.0235) (end 119.142708 75.25) (width 0.254) (layer "F.Cu") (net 6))
 (via (at 119.369208 75.0235) (size 0.8) (drill 0.4) (layers "F.Cu" "B.Cu") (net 6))
 (via (at 119.369208 76.4765) (size 0.8) (drill 0.4) (layers "F.Cu" "B.Cu") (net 6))
 (segment (start 119.369208 76.4765) (end 119.369208 75.0235) (width 0.254) (layer "B.Cu") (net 6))
 (segment (start 117.38 75.75) (end 116.501 75.75) (width 0.254) (layer "F.Cu") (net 5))
 (segment (start 116.501 75.75) (end 116.478 75.773) (width 0.254) (layer "F.Cu") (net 5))
 (segment (start 116.478 76.727) (end 116.501 76.75) (width 0.254) (layer "F.Cu") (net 5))
 (segment (start 116.478 75.773) (end 116.478 76.727) (width 0.254) (layer "F.Cu") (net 5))
 (segment (start 117.38 75.75) (end 122.2875 75.75) (width 0.254) (layer "F.Cu") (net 5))
 (segment (start 122.2875 75.75) (end 123.2875 74.75) (width 0.254) (layer "F.Cu") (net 5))
 (segment (start 116.501 76.75) (end 117.38 76.75) (width 0.254) (layer "F.Cu") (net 5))
 (segment (start 117.38 71.72) (end 117.4 71.7) (width 0.6) (layer "F.Cu") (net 2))
 (segment (start 117.38 72.8) (end 117.38 71.72) (width 0.6) (layer "F.Cu") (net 2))
 (segment (start 122.8 78.275) (end 122.225 78.275) (width 0.4) (layer "F.Cu") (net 2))
 (segment (start 117.38 80.22) (end 117.3 80.3) (width 0.6) (layer "F.Cu") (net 2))
 (segment (start 123.2875 78.0125) (end 123.025 78.275) (width 0.4) (layer "F.Cu") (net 2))
 (segment (start 123.2875 77.25) (end 123.2875 78.0125) (width 0.4) (layer "F.Cu") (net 2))
 (segment (start 123.025 78.275) (end 122.8 78.275) (width 0.4) (layer "F.Cu") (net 2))
 (segment (start 117.38 79.2) (end 117.38 80.22) (width 0.6) (layer "F.Cu") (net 2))
 (via (at 120.4 76.9765) (size 0.8) (drill 0.4) (layers "F.Cu" "B.Cu") (free) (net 2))
 (via (at 125.8 78.8) (size 0.8) (drill 0.4) (layers "F.Cu" "B.Cu") (free) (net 2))
 (via (at 125.8 73.3) (size 0.8) (drill 0.4) (layers "F.Cu" "B.Cu") (free) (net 2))
 (via (at 116 74.3) (size 0.8) (drill 0.4) (layers "F.Cu" "B.Cu") (free) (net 2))
 (via (at 115.6 76) (size 0.8) (drill 0.4) (layers "F.Cu" "B.Cu") (free) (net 2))
 (via (at 120.4 75.0235) (size 0.8) (drill 0.4) (layers "F.Cu" "B.Cu") (free) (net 2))
 (via (at 116 77.7) (size 0.8) (drill 0.4) (layers "F.Cu" "B.Cu") (free) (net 2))
 (segment (start 118.55 74.75) (end 119.575 73.725) (width 0.254) (layer "F.Cu") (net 4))
 (segment (start 117.38 74.75) (end 118.55 74.75) (width 0.254) (layer "F.Cu") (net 4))
 (segment (start 119.575 73.725) (end 119.575 73.7) (width 0.254) (layer "F.Cu") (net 4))
 (segment (start 119.325 77.75) (end 119.575 78) (width 0.254) (layer "F.Cu") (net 1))
 (segment (start 117.38 77.75) (end 119.325 77.75) (width 0.254) (layer "F.Cu") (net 1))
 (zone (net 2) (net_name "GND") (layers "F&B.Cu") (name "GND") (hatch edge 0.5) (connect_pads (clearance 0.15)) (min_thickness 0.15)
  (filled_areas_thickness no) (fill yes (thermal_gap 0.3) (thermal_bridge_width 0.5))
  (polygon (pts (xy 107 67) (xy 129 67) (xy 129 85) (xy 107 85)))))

